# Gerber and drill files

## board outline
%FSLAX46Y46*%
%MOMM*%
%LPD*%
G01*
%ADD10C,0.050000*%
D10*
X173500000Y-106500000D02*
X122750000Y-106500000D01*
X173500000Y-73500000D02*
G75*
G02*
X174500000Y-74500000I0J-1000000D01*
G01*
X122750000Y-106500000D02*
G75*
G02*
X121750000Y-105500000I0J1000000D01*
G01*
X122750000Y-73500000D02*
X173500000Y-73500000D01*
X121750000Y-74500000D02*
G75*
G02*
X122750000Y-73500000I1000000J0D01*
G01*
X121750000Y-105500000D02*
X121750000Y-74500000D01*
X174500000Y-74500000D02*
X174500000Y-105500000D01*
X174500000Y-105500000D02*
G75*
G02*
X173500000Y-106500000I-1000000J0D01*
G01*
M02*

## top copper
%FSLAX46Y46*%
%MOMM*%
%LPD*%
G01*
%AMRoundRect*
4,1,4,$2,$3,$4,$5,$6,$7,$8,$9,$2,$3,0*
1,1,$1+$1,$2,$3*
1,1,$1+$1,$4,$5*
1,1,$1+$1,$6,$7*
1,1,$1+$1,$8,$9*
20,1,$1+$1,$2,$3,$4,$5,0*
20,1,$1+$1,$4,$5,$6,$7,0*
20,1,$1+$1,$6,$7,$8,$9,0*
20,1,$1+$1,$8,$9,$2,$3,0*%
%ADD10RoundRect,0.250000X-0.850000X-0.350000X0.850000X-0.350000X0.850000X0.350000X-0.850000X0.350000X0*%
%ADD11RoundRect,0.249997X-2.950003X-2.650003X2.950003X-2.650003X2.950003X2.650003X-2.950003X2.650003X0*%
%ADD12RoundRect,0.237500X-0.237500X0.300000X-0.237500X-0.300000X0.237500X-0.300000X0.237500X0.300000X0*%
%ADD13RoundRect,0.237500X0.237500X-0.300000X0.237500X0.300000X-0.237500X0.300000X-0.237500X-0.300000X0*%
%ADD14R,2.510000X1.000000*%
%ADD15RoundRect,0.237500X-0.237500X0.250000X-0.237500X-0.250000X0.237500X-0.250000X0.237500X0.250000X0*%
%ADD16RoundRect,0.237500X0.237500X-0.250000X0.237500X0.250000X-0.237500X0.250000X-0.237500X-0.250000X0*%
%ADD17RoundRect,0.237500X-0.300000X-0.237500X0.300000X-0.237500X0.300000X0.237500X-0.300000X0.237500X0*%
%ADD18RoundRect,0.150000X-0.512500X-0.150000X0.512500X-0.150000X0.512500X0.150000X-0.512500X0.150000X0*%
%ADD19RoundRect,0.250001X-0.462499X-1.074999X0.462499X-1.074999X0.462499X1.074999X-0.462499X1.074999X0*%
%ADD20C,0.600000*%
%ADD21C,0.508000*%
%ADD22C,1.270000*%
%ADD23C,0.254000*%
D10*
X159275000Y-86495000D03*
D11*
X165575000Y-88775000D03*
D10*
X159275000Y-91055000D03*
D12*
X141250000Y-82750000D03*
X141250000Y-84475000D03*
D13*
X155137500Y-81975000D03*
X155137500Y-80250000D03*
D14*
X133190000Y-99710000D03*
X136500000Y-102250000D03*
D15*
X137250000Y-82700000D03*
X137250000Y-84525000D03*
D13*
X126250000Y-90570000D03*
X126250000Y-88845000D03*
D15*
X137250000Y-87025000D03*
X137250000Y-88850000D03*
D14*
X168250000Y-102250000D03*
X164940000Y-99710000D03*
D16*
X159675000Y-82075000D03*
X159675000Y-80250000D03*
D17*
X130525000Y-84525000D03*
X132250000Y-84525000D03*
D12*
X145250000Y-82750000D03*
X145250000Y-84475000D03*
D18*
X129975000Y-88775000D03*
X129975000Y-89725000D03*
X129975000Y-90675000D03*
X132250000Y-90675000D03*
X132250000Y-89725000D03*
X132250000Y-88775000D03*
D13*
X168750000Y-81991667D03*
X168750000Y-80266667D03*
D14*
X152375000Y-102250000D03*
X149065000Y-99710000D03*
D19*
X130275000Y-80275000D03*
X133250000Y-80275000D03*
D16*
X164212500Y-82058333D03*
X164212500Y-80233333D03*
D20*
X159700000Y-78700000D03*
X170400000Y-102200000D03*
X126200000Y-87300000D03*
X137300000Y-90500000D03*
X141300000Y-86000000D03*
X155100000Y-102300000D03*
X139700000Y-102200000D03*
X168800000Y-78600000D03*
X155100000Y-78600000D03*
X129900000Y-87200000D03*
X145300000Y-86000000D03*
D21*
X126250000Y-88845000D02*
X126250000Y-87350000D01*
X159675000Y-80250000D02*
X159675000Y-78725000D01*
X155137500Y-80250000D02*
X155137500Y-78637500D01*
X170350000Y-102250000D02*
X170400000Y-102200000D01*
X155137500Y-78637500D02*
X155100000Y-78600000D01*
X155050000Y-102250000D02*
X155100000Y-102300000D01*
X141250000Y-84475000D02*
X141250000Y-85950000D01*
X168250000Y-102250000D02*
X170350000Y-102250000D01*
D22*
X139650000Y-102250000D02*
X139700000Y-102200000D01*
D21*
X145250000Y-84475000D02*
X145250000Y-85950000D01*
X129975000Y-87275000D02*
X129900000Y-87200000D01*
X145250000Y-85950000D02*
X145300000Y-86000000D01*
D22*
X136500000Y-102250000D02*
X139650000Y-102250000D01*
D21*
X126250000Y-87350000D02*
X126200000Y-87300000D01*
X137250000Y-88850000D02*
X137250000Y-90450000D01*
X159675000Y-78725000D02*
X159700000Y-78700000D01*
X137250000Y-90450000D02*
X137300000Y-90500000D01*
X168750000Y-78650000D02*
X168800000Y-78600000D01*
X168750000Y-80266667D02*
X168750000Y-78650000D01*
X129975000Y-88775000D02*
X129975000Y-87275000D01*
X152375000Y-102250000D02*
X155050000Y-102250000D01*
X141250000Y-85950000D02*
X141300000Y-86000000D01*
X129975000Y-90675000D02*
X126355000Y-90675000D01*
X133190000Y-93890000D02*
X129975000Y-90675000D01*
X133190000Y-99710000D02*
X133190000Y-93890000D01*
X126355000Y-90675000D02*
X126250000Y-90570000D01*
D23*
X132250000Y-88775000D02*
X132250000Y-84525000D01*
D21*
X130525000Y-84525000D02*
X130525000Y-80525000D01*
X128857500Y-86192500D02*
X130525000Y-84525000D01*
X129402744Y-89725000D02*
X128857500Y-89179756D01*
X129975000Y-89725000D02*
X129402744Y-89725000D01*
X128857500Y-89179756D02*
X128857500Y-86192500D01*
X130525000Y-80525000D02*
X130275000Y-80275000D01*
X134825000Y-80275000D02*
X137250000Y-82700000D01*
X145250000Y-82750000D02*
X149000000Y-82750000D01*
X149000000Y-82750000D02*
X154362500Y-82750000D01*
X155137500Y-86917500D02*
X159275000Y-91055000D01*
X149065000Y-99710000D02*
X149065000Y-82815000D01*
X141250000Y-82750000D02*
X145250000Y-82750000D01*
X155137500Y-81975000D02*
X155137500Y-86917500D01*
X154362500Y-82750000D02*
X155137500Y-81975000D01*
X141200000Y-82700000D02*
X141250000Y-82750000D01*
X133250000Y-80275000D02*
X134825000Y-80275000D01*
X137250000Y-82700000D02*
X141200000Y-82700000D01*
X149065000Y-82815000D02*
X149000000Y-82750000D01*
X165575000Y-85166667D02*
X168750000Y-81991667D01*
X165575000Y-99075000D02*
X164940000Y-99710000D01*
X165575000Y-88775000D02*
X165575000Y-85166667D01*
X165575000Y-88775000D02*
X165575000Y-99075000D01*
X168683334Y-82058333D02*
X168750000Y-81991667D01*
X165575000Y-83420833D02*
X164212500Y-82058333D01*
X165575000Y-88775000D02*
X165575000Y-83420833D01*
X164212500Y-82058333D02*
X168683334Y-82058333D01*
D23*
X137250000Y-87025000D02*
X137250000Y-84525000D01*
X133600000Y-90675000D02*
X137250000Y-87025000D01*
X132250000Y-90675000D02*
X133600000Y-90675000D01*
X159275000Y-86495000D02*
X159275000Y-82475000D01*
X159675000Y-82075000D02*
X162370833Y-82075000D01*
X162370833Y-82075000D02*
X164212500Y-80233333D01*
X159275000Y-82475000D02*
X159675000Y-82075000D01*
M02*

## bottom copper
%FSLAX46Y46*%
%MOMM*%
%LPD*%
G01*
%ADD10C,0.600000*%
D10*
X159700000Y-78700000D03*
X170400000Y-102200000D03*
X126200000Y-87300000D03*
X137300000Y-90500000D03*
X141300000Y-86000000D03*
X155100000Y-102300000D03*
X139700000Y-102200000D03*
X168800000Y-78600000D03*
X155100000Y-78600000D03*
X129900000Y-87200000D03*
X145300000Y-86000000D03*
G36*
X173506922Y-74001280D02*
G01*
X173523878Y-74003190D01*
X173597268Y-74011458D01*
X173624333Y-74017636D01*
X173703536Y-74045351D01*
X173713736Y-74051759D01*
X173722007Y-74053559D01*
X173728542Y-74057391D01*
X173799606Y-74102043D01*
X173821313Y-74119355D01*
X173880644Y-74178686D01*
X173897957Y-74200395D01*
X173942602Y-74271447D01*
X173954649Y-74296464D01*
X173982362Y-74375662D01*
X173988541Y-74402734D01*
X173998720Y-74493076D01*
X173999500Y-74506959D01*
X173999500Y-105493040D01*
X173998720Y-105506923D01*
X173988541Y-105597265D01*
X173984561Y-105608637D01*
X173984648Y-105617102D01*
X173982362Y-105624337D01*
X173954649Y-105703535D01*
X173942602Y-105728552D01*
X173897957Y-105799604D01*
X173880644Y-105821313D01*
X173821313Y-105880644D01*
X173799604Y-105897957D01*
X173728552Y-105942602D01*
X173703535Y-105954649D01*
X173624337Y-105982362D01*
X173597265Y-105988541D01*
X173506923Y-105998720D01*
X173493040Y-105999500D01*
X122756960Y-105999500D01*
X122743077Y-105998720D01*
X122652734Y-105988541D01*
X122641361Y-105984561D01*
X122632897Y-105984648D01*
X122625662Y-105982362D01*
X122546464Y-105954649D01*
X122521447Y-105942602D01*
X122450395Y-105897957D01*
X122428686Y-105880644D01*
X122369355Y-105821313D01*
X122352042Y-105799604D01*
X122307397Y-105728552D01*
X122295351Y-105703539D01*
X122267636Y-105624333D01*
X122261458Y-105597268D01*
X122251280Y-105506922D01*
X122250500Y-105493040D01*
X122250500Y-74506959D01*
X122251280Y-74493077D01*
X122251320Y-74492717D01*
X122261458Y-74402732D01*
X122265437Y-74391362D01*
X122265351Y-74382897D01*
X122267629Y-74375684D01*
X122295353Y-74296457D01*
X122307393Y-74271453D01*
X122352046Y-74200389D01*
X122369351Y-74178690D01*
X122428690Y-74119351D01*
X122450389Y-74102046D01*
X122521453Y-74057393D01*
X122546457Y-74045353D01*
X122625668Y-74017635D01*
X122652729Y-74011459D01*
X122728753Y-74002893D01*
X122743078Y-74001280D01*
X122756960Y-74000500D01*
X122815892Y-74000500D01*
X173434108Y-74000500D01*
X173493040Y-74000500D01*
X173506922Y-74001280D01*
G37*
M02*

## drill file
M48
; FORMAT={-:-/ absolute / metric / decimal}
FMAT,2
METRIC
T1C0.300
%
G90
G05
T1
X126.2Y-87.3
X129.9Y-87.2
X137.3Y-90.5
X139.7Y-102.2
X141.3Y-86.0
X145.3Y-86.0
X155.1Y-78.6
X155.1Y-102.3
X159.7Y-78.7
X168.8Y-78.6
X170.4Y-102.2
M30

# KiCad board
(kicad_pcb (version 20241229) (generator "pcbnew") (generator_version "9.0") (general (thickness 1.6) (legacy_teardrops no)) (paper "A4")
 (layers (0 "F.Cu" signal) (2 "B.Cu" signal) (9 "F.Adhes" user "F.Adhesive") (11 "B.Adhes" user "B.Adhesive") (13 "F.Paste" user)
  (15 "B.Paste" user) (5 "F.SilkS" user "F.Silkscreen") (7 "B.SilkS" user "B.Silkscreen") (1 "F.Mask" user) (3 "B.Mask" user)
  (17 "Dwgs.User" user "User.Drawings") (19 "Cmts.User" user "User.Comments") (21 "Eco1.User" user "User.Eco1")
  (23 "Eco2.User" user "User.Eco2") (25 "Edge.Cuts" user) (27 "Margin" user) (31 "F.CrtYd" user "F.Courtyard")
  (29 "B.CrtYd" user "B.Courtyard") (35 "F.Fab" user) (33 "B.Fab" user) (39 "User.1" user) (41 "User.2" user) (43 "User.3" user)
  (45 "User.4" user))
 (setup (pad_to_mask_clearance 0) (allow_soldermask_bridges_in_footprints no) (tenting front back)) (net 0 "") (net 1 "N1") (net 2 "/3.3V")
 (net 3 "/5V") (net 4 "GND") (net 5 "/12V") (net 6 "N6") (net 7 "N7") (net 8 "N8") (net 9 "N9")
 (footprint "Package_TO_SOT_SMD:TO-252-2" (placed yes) (layer "F.Cu") (at 164.315 88.775)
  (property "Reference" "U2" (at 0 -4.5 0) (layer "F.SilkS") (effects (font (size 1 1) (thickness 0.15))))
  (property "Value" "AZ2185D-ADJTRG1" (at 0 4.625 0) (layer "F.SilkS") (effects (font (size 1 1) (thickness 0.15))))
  (pad "" smd roundrect (at -0.415 -1.525) (size 3.05 2.75) (layers "F.Paste") (roundrect_rratio 0.090909))
  (pad "" smd roundrect (at -0.415 1.525) (size 3.05 2.75) (layers "F.Paste") (roundrect_rratio 0.090909))
  (pad "" smd roundrect (at 2.935 -1.525) (size 3.05 2.75) (layers "F.Paste") (roundrect_rratio 0.090909))
  (pad "" smd roundrect (at 2.935 1.525) (size 3.05 2.75) (layers "F.Paste") (roundrect_rratio 0.090909))
  (pad "1" smd roundrect (at -5.04 -2.28) (size 2.2 1.2) (layers "F.Cu" "F.Mask" "F.Paste") (roundrect_rratio 0.208333) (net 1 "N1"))
  (pad "2" smd roundrect (at 1.26 0) (size 6.4 5.8) (layers "F.Cu" "F.Mask") (roundrect_rratio 0.043103) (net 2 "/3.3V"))
  (pad "3" smd roundrect (at -5.04 2.28) (size 2.2 1.2) (layers "F.Cu" "F.Mask" "F.Paste") (roundrect_rratio 0.208333) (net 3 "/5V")))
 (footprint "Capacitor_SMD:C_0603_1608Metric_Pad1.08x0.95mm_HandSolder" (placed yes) (layer "F.Cu") (at 141.25 83.6125 -90)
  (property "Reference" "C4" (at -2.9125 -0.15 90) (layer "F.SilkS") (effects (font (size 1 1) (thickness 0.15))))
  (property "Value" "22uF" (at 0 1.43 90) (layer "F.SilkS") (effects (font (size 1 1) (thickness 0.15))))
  (pad "1" smd roundrect (at -0.8625 0 270) (size 1.075 0.95) (layers "F.Cu" "F.Mask" "F.Paste") (roundrect_rratio 0.25) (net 3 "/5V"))
  (pad "2" smd roundrect (at 0.8625 0 270) (size 1.075 0.95) (layers "F.Cu" "F.Mask" "F.Paste") (roundrect_rratio 0.25) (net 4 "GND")))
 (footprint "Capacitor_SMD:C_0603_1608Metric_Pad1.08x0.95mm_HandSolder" (layer "F.Cu") (at 155.1375 81.1125 90)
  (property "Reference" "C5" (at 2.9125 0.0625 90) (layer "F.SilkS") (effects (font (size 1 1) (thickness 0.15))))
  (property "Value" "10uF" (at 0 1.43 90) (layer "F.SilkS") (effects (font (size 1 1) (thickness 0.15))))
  (pad "1" smd roundrect (at -0.8625 0 90) (size 1.075 0.95) (layers "F.Cu" "F.Mask" "F.Paste") (roundrect_rratio 0.25) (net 3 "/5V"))
  (pad "2" smd roundrect (at 0.8625 0 90) (size 1.075 0.95) (layers "F.Cu" "F.Mask" "F.Paste") (roundrect_rratio 0.25) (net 4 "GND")))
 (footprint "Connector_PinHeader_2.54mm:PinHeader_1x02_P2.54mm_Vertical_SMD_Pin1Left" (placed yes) (layer "F.Cu") (at 134.845 100.98)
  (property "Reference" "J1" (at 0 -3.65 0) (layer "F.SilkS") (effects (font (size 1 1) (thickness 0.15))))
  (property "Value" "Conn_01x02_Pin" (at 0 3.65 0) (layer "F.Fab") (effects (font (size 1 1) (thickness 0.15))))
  (pad "1" smd rect (at -1.655 -1.27) (size 2.51 1) (layers "F.Cu" "F.Mask" "F.Paste") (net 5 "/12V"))
  (pad "2" smd rect (at 1.655 1.27) (size 2.51 1) (layers "F.Cu" "F.Mask" "F.Paste") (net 4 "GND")))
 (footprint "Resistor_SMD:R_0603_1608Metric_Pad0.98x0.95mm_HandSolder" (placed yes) (layer "F.Cu") (at 137.25 83.6125 -90)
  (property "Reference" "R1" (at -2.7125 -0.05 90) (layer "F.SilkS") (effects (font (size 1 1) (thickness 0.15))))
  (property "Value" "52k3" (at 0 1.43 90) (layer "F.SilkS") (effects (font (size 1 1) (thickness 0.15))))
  (pad "1" smd roundrect (at -0.9125 0 270) (size 0.975 0.95) (layers "F.Cu" "F.Mask" "F.Paste") (roundrect_rratio 0.25) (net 3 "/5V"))
  (pad "2" smd roundrect (at 0.9125 0 270) (size 0.975 0.95) (layers "F.Cu" "F.Mask" "F.Paste") (roundrect_rratio 0.25) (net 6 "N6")))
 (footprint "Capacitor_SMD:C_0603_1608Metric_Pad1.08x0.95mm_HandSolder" (layer "F.Cu") (at 126.25 89.7075 90)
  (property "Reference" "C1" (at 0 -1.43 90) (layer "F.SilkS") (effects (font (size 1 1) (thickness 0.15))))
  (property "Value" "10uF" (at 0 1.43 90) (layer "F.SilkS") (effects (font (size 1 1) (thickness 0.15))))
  (pad "1" smd roundrect (at -0.8625 0 90) (size 1.075 0.95) (layers "F.Cu" "F.Mask" "F.Paste") (roundrect_rratio 0.25) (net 5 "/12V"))
  (pad "2" smd roundrect (at 0.8625 0 90) (size 1.075 0.95) (layers "F.Cu" "F.Mask" "F.Paste") (roundrect_rratio 0.25) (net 4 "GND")))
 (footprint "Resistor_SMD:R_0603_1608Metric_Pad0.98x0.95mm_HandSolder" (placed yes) (layer "F.Cu") (at 137.25 87.9375 -90)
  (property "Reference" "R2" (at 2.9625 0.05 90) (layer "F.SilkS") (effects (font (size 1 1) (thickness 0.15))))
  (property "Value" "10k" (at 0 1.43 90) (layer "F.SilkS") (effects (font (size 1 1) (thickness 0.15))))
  (pad "1" smd roundrect (at -0.9125 0 270) (size 0.975 0.95) (layers "F.Cu" "F.Mask" "F.Paste") (roundrect_rratio 0.25) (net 6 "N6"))
  (pad "2" smd roundrect (at 0.9125 0 270) (size 0.975 0.95) (layers "F.Cu" "F.Mask" "F.Paste") (roundrect_rratio 0.25) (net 4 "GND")))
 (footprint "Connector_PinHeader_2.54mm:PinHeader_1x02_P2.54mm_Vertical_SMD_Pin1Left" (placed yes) (layer "F.Cu") (at 166.595 100.98 180)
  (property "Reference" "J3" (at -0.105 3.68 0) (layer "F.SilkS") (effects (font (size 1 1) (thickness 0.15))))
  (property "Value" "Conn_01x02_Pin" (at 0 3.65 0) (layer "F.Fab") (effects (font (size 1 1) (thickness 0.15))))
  (pad "1" smd rect (at -1.655 -1.27 180) (size 2.51 1) (layers "F.Cu" "F.Mask" "F.Paste") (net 4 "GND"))
  (pad "2" smd rect (at 1.655 1.27 180) (size 2.51 1) (layers "F.Cu" "F.Mask" "F.Paste") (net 2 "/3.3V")))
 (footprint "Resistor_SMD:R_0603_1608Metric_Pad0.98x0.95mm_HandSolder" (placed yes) (layer "F.Cu") (at 159.675 81.1625 90)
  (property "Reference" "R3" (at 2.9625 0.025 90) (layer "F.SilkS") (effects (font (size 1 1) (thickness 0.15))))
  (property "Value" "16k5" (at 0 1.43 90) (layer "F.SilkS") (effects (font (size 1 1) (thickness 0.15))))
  (pad "1" smd roundrect (at -0.9125 0 90) (size 0.975 0.95) (layers "F.Cu" "F.Mask" "F.Paste") (roundrect_rratio 0.25) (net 1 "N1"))
  (pad "2" smd roundrect (at 0.9125 0 90) (size 0.975 0.95) (layers "F.Cu" "F.Mask" "F.Paste") (roundrect_rratio 0.25) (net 4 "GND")))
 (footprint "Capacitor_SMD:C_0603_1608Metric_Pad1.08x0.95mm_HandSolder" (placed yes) (layer "F.Cu") (at 131.3875 84.525)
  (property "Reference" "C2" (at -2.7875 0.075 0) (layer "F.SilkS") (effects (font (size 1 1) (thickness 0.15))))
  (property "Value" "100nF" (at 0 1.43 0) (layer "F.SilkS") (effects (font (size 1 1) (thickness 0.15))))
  (pad "1" smd roundrect (at -0.8625 0) (size 1.075 0.95) (layers "F.Cu" "F.Mask" "F.Paste") (roundrect_rratio 0.25) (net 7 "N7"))
  (pad "2" smd roundrect (at 0.8625 0) (size 1.075 0.95) (layers "F.Cu" "F.Mask" "F.Paste") (roundrect_rratio 0.25) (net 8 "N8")))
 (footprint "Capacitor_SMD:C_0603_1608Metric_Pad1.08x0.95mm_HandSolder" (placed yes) (layer "F.Cu") (at 145.25 83.6125 -90)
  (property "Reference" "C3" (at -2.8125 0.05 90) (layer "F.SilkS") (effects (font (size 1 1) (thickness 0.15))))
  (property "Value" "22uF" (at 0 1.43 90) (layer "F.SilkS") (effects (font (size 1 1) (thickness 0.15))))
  (pad "1" smd roundrect (at -0.8625 0 270) (size 1.075 0.95) (layers "F.Cu" "F.Mask" "F.Paste") (roundrect_rratio 0.25) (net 3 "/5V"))
  (pad "2" smd roundrect (at 0.8625 0 270) (size 1.075 0.95) (layers "F.Cu" "F.Mask" "F.Paste") (roundrect_rratio 0.25) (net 4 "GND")))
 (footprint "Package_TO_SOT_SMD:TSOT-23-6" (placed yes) (layer "F.Cu") (at 131.1125 89.725)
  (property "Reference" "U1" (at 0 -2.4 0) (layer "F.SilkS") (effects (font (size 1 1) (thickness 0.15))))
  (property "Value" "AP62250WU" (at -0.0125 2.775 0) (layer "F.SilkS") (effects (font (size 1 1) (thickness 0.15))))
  (pad "1" smd roundrect (at -1.1375 -0.95) (size 1.325 0.6) (layers "F.Cu" "F.Mask" "F.Paste") (roundrect_rratio 0.25) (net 4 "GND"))
  (pad "2" smd roundrect (at -1.1375 0) (size 1.325 0.6) (layers "F.Cu" "F.Mask" "F.Paste") (roundrect_rratio 0.25) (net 7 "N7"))
  (pad "3" smd roundrect (at -1.1375 0.95) (size 1.325 0.6) (layers "F.Cu" "F.Mask" "F.Paste") (roundrect_rratio 0.25) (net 5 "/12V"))
  (pad "4" smd roundrect (at 1.1375 0.95) (size 1.325 0.6) (layers "F.Cu" "F.Mask" "F.Paste") (roundrect_rratio 0.25) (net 6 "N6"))
  (pad "5" smd roundrect (at 1.1375 0) (size 1.325 0.6) (layers "F.Cu" "F.Mask" "F.Paste") (roundrect_rratio 0.25) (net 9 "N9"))
  (pad "6" smd roundrect (at 1.1375 -0.95) (size 1.325 0.6) (layers "F.Cu" "F.Mask" "F.Paste") (roundrect_rratio 0.25) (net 8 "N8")))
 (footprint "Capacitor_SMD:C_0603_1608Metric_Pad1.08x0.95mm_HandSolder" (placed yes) (layer "F.Cu") (at 168.75 81.129167 90)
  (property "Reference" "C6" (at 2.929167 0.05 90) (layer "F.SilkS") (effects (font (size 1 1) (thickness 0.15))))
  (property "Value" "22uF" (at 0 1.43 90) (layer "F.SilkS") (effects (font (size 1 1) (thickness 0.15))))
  (pad "1" smd roundrect (at -0.8625 0 90) (size 1.075 0.95) (layers "F.Cu" "F.Mask" "F.Paste") (roundrect_rratio 0.25) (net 2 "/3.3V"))
  (pad "2" smd roundrect (at 0.8625 0 90) (size 1.075 0.95) (layers "F.Cu" "F.Mask" "F.Paste") (roundrect_rratio 0.25) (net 4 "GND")))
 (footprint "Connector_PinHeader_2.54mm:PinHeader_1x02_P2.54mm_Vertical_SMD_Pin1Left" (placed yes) (layer "F.Cu") (at 150.72 100.98 180)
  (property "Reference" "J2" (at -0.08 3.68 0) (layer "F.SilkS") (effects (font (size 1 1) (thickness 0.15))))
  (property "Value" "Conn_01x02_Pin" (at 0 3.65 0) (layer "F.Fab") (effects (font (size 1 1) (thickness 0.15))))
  (pad "1" smd rect (at -1.655 -1.27 180) (size 2.51 1) (layers "F.Cu" "F.Mask" "F.Paste") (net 4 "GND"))
  (pad "2" smd rect (at 1.655 1.27 180) (size 2.51 1) (layers "F.Cu" "F.Mask" "F.Paste") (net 3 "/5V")))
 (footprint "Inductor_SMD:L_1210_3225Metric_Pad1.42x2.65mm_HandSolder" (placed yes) (layer "F.Cu") (at 131.7625 80.275)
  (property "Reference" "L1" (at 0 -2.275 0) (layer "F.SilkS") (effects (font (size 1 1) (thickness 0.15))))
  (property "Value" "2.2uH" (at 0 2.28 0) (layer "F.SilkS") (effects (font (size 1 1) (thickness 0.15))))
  (pad "1" smd roundrect (at -1.4875 0) (size 1.425 2.65) (layers "F.Cu" "F.Mask" "F.Paste") (roundrect_rratio 0.175439) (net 7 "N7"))
  (pad "2" smd roundrect (at 1.4875 0) (size 1.425 2.65) (layers "F.Cu" "F.Mask" "F.Paste") (roundrect_rratio 0.175439) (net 3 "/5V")))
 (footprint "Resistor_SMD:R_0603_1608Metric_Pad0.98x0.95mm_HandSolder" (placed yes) (layer "F.Cu") (at 164.2125 81.145833 90)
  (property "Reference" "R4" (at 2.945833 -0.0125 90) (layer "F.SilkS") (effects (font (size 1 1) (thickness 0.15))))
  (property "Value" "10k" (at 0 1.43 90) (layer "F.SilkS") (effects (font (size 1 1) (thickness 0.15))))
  (pad "1" smd roundrect (at -0.9125 0 90) (size 0.975 0.95) (layers "F.Cu" "F.Mask" "F.Paste") (roundrect_rratio 0.25) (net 2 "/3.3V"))
  (pad "2" smd roundrect (at 0.9125 0 90) (size 0.975 0.95) (layers "F.Cu" "F.Mask" "F.Paste") (roundrect_rratio 0.25) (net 1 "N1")))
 (gr_line (start 173.5 106.5) (end 122.75 106.5) (stroke (width 0.05) (type default)) (layer "Edge.Cuts"))
 (gr_arc (start 173.5 73.5) (mid 174.207107 73.792893) (end 174.5 74.5) (stroke (width 0.05) (type default)) (layer "Edge.Cuts"))
 (gr_arc (start 122.75 106.5) (mid 122.042893 106.207107) (end 121.75 105.5) (stroke (width 0.05) (type default)) (layer "Edge.Cuts"))
 (gr_line (start 122.75 73.5) (end 173.5 73.5) (stroke (width 0.05) (type default)) (layer "Edge.Cuts"))
 (gr_arc (start 121.75 74.5) (mid 122.042893 73.792893) (end 122.75 73.5) (stroke (width 0.05) (type default)) (layer "Edge.Cuts"))
 (gr_line (start 121.75 105.5) (end 121.75 74.5) (stroke (width 0.05) (type default)) (layer "Edge.Cuts"))
 (gr_line (start 174.5 74.5) (end 174.5 105.5) (stroke (width 0.05) (type default)) (layer "Edge.Cuts"))
 (gr_arc (start 174.5 105.5) (mid 174.207107 106.207107) (end 173.5 106.5) (stroke (width 0.05) (type default)) (layer "Edge.Cuts"))
 (segment (start 126.25 88.845) (end 126.25 87.35) (width 0.508) (layer "F.Cu") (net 4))
 (segment (start 159.675 80.25) (end 159.675 78.725) (width 0.508) (layer "F.Cu") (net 4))
 (segment (start 155.1375 80.25) (end 155.1375 78.6375) (width 0.508) (layer "F.Cu") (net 4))
 (segment (start 170.35 102.25) (end 170.4 102.2) (width 0.508) (layer "F.Cu") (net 4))
 (segment (start 155.1375 78.6375) (end 155.1 78.6) (width 0.508) (layer "F.Cu") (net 4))
 (segment (start 155.05 102.25) (end 155.1 102.3) (width 0.508) (layer "F.Cu") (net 4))
 (segment (start 141.25 84.475) (end 141.25 85.95) (width 0.508) (layer "F.Cu") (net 4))
 (segment (start 168.25 102.25) (end 170.35 102.25) (width 0.508) (layer "F.Cu") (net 4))
 (segment (start 139.65 102.25) (end 139.7 102.2) (width 1.27) (layer "F.Cu") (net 4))
 (segment (start 145.25 84.475) (end 145.25 85.95) (width 0.508) (layer "F.Cu") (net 4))
 (segment (start 129.975 87.275) (end 129.9 87.2) (width 0.508) (layer "F.Cu") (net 4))
 (segment (start 145.25 85.95) (end 145.3 86) (width 0.508) (layer "F.Cu") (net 4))
 (segment (start 136.5 102.25) (end 139.65 102.25) (width 1.27) (layer "F.Cu") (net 4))
 (segment (start 126.25 87.35) (end 126.2 87.3) (width 0.508) (layer "F.Cu") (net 4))
 (segment (start 137.25 88.85) (end 137.25 90.45) (width 0.508) (layer "F.Cu") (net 4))
 (segment (start 159.675 78.725) (end 159.7 78.7) (width 0.508) (layer "F.Cu") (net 4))
 (segment (start 137.25 90.45) (end 137.3 90.5) (width 0.508) (layer "F.Cu") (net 4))
 (segment (start 168.75 78.65) (end 168.8 78.6) (width 0.508) (layer "F.Cu") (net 4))
 (segment (start 168.75 80.266667) (end 168.75 78.65) (width 0.508) (layer "F.Cu") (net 4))
 (segment (start 129.975 88.775) (end 129.975 87.275) (width 0.508) (layer "F.Cu") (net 4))
 (segment (start 152.375 102.25) (end 155.05 102.25) (width 0.508) (layer "F.Cu") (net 4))
 (segment (start 141.25 85.95) (end 141.3 86) (width 0.508) (layer "F.Cu") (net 4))
 (via (at 159.7 78.7) (size 0.6) (drill 0.3) (layers "F.Cu" "B.Cu") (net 4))
 (via (at 170.4 102.2) (size 0.6) (drill 0.3) (layers "F.Cu" "B.Cu") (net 4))
 (via (at 126.2 87.3) (size 0.6) (drill 0.3) (layers "F.Cu" "B.Cu") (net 4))
 (via (at 137.3 90.5) (size 0.6) (drill 0.3) (layers "F.Cu" "B.Cu") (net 4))
 (via (at 141.3 86) (size 0.6) (drill 0.3) (layers "F.Cu" "B.Cu") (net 4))
 (via (at 155.1 102.3) (size 0.6) (drill 0.3) (layers "F.Cu" "B.Cu") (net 4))
 (via (at 139.7 102.2) (size 0.6) (drill 0.3) (layers "F.Cu" "B.Cu") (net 4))
 (via (at 168.8 78.6) (size 0.6) (drill 0.3) (layers "F.Cu" "B.Cu") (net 4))
 (via (at 155.1 78.6) (size 0.6) (drill 0.3) (layers "F.Cu" "B.Cu") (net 4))
 (via (at 129.9 87.2) (size 0.6) (drill 0.3) (layers "F.Cu" "B.Cu") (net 4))
 (via (at 145.3 86) (size 0.6) (drill 0.3) (layers "F.Cu" "B.Cu") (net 4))
 (segment (start 129.975 90.675) (end 126.355 90.675) (width 0.508) (layer "F.Cu") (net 5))
 (segment (start 133.19 93.89) (end 129.975 90.675) (width 0.508) (layer "F.Cu") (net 5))
 (segment (start 133.19 99.71) (end 133.19 93.89) (width 0.508) (layer "F.Cu") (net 5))
 (segment (start 126.355 90.675) (end 126.25 90.57) (width 0.508) (layer "F.Cu") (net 5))
 (segment (start 132.25 88.775) (end 132.25 84.525) (width 0.254) (layer "F.Cu") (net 8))
 (segment (start 130.525 84.525) (end 130.525 80.525) (width 0.508) (layer "F.Cu") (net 7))
 (segment (start 128.8575 86.1925) (end 130.525 84.525) (width 0.508) (layer "F.Cu") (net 7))
 (segment (start 129.402744 89.725) (end 128.8575 89.179756) (width 0.508) (layer "F.Cu") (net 7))
 (segment (start 129.975 89.725) (end 129.402744 89.725) (width 0.508) (layer "F.Cu") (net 7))
 (segment (start 128.8575 89.179756) (end 128.8575 86.1925) (width 0.508) (layer "F.Cu") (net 7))
 (segment (start 130.525 80.525) (end 130.275 80.275) (width 0.508) (layer "F.Cu") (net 7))
 (segment (start 134.825 80.275) (end 137.25 82.7) (width 0.508) (layer "F.Cu") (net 3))
 (segment (start 145.25 82.75) (end 149 82.75) (width 0.508) (layer "F.Cu") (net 3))
 (segment (start 149 82.75) (end 154.3625 82.75) (width 0.508) (layer "F.Cu") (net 3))
 (segment (start 155.1375 86.9175) (end 159.275 91.055) (width 0.508) (layer "F.Cu") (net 3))
 (segment (start 149.065 99.71) (end 149.065 82.815) (width 0.508) (layer "F.Cu") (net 3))
 (segment (start 141.25 82.75) (end 145.25 82.75) (width 0.508) (layer "F.Cu") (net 3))
 (segment (start 155.1375 81.975) (end 155.1375 86.9175) (width 0.508) (layer "F.Cu") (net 3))
 (segment (start 154.3625 82.75) (end 155.1375 81.975) (width 0.508) (layer "F.Cu") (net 3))
 (segment (start 141.2 82.7) (end 141.25 82.75) (width 0.508) (layer "F.Cu") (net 3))
 (segment (start 133.25 80.275) (end 134.825 80.275) (width 0.508) (layer "F.Cu") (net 3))
 (segment (start 137.25 82.7) (end 141.2 82.7) (width 0.508) (layer "F.Cu") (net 3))
 (segment (start 149.065 82.815) (end 149 82.75) (width 0.508) (layer "F.Cu") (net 3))
 (segment (start 165.575 85.166667) (end 168.75 81.991667) (width 0.508) (layer "F.Cu") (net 2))
 (segment (start 165.575 99.075) (end 164.94 99.71) (width 0.508) (layer "F.Cu") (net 2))
 (segment (start 165.575 88.775) (end 165.575 85.166667) (width 0.508) (layer "F.Cu") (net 2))
 (segment (start 165.575 88.775) (end 165.575 99.075) (width 0.508) (layer "F.Cu") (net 2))
 (segment (start 168.683334 82.058333) (end 168.75 81.991667) (width 0.508) (layer "F.Cu") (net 2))
 (segment (start 165.575 83.420833) (end 164.2125 82.058333) (width 0.508) (layer "F.Cu") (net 2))
 (segment (start 165.575 88.775) (end 165.575 83.420833) (width 0.508) (layer "F.Cu") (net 2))
 (segment (start 164.2125 82.058333) (end 168.683334 82.058333) (width 0.508) (layer "F.Cu") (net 2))
 (segment (start 137.25 87.025) (end 137.25 84.525) (width 0.254) (layer "F.Cu") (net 6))
 (segment (start 133.6 90.675) (end 137.25 87.025) (width 0.254) (layer "F.Cu") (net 6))
 (segment (start 132.25 90.675) (end 133.6 90.675) (width 0.254) (layer "F.Cu") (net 6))
 (segment (start 159.275 86.495) (end 159.275 82.475) (width 0.254) (layer "F.Cu") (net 1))
 (segment (start 159.675 82.075) (end 162.370833 82.075) (width 0.254) (layer "F.Cu") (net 1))
 (segment (start 162.370833 82.075) (end 164.2125 80.233333) (width 0.254) (layer "F.Cu") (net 1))
 (segment (start 159.275 82.475) (end 159.675 82.075) (width 0.254) (layer "F.Cu") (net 1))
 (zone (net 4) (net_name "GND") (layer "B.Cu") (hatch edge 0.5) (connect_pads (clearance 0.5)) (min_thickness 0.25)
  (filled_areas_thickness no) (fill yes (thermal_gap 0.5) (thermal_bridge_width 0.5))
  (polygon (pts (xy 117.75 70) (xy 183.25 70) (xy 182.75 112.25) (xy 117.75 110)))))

